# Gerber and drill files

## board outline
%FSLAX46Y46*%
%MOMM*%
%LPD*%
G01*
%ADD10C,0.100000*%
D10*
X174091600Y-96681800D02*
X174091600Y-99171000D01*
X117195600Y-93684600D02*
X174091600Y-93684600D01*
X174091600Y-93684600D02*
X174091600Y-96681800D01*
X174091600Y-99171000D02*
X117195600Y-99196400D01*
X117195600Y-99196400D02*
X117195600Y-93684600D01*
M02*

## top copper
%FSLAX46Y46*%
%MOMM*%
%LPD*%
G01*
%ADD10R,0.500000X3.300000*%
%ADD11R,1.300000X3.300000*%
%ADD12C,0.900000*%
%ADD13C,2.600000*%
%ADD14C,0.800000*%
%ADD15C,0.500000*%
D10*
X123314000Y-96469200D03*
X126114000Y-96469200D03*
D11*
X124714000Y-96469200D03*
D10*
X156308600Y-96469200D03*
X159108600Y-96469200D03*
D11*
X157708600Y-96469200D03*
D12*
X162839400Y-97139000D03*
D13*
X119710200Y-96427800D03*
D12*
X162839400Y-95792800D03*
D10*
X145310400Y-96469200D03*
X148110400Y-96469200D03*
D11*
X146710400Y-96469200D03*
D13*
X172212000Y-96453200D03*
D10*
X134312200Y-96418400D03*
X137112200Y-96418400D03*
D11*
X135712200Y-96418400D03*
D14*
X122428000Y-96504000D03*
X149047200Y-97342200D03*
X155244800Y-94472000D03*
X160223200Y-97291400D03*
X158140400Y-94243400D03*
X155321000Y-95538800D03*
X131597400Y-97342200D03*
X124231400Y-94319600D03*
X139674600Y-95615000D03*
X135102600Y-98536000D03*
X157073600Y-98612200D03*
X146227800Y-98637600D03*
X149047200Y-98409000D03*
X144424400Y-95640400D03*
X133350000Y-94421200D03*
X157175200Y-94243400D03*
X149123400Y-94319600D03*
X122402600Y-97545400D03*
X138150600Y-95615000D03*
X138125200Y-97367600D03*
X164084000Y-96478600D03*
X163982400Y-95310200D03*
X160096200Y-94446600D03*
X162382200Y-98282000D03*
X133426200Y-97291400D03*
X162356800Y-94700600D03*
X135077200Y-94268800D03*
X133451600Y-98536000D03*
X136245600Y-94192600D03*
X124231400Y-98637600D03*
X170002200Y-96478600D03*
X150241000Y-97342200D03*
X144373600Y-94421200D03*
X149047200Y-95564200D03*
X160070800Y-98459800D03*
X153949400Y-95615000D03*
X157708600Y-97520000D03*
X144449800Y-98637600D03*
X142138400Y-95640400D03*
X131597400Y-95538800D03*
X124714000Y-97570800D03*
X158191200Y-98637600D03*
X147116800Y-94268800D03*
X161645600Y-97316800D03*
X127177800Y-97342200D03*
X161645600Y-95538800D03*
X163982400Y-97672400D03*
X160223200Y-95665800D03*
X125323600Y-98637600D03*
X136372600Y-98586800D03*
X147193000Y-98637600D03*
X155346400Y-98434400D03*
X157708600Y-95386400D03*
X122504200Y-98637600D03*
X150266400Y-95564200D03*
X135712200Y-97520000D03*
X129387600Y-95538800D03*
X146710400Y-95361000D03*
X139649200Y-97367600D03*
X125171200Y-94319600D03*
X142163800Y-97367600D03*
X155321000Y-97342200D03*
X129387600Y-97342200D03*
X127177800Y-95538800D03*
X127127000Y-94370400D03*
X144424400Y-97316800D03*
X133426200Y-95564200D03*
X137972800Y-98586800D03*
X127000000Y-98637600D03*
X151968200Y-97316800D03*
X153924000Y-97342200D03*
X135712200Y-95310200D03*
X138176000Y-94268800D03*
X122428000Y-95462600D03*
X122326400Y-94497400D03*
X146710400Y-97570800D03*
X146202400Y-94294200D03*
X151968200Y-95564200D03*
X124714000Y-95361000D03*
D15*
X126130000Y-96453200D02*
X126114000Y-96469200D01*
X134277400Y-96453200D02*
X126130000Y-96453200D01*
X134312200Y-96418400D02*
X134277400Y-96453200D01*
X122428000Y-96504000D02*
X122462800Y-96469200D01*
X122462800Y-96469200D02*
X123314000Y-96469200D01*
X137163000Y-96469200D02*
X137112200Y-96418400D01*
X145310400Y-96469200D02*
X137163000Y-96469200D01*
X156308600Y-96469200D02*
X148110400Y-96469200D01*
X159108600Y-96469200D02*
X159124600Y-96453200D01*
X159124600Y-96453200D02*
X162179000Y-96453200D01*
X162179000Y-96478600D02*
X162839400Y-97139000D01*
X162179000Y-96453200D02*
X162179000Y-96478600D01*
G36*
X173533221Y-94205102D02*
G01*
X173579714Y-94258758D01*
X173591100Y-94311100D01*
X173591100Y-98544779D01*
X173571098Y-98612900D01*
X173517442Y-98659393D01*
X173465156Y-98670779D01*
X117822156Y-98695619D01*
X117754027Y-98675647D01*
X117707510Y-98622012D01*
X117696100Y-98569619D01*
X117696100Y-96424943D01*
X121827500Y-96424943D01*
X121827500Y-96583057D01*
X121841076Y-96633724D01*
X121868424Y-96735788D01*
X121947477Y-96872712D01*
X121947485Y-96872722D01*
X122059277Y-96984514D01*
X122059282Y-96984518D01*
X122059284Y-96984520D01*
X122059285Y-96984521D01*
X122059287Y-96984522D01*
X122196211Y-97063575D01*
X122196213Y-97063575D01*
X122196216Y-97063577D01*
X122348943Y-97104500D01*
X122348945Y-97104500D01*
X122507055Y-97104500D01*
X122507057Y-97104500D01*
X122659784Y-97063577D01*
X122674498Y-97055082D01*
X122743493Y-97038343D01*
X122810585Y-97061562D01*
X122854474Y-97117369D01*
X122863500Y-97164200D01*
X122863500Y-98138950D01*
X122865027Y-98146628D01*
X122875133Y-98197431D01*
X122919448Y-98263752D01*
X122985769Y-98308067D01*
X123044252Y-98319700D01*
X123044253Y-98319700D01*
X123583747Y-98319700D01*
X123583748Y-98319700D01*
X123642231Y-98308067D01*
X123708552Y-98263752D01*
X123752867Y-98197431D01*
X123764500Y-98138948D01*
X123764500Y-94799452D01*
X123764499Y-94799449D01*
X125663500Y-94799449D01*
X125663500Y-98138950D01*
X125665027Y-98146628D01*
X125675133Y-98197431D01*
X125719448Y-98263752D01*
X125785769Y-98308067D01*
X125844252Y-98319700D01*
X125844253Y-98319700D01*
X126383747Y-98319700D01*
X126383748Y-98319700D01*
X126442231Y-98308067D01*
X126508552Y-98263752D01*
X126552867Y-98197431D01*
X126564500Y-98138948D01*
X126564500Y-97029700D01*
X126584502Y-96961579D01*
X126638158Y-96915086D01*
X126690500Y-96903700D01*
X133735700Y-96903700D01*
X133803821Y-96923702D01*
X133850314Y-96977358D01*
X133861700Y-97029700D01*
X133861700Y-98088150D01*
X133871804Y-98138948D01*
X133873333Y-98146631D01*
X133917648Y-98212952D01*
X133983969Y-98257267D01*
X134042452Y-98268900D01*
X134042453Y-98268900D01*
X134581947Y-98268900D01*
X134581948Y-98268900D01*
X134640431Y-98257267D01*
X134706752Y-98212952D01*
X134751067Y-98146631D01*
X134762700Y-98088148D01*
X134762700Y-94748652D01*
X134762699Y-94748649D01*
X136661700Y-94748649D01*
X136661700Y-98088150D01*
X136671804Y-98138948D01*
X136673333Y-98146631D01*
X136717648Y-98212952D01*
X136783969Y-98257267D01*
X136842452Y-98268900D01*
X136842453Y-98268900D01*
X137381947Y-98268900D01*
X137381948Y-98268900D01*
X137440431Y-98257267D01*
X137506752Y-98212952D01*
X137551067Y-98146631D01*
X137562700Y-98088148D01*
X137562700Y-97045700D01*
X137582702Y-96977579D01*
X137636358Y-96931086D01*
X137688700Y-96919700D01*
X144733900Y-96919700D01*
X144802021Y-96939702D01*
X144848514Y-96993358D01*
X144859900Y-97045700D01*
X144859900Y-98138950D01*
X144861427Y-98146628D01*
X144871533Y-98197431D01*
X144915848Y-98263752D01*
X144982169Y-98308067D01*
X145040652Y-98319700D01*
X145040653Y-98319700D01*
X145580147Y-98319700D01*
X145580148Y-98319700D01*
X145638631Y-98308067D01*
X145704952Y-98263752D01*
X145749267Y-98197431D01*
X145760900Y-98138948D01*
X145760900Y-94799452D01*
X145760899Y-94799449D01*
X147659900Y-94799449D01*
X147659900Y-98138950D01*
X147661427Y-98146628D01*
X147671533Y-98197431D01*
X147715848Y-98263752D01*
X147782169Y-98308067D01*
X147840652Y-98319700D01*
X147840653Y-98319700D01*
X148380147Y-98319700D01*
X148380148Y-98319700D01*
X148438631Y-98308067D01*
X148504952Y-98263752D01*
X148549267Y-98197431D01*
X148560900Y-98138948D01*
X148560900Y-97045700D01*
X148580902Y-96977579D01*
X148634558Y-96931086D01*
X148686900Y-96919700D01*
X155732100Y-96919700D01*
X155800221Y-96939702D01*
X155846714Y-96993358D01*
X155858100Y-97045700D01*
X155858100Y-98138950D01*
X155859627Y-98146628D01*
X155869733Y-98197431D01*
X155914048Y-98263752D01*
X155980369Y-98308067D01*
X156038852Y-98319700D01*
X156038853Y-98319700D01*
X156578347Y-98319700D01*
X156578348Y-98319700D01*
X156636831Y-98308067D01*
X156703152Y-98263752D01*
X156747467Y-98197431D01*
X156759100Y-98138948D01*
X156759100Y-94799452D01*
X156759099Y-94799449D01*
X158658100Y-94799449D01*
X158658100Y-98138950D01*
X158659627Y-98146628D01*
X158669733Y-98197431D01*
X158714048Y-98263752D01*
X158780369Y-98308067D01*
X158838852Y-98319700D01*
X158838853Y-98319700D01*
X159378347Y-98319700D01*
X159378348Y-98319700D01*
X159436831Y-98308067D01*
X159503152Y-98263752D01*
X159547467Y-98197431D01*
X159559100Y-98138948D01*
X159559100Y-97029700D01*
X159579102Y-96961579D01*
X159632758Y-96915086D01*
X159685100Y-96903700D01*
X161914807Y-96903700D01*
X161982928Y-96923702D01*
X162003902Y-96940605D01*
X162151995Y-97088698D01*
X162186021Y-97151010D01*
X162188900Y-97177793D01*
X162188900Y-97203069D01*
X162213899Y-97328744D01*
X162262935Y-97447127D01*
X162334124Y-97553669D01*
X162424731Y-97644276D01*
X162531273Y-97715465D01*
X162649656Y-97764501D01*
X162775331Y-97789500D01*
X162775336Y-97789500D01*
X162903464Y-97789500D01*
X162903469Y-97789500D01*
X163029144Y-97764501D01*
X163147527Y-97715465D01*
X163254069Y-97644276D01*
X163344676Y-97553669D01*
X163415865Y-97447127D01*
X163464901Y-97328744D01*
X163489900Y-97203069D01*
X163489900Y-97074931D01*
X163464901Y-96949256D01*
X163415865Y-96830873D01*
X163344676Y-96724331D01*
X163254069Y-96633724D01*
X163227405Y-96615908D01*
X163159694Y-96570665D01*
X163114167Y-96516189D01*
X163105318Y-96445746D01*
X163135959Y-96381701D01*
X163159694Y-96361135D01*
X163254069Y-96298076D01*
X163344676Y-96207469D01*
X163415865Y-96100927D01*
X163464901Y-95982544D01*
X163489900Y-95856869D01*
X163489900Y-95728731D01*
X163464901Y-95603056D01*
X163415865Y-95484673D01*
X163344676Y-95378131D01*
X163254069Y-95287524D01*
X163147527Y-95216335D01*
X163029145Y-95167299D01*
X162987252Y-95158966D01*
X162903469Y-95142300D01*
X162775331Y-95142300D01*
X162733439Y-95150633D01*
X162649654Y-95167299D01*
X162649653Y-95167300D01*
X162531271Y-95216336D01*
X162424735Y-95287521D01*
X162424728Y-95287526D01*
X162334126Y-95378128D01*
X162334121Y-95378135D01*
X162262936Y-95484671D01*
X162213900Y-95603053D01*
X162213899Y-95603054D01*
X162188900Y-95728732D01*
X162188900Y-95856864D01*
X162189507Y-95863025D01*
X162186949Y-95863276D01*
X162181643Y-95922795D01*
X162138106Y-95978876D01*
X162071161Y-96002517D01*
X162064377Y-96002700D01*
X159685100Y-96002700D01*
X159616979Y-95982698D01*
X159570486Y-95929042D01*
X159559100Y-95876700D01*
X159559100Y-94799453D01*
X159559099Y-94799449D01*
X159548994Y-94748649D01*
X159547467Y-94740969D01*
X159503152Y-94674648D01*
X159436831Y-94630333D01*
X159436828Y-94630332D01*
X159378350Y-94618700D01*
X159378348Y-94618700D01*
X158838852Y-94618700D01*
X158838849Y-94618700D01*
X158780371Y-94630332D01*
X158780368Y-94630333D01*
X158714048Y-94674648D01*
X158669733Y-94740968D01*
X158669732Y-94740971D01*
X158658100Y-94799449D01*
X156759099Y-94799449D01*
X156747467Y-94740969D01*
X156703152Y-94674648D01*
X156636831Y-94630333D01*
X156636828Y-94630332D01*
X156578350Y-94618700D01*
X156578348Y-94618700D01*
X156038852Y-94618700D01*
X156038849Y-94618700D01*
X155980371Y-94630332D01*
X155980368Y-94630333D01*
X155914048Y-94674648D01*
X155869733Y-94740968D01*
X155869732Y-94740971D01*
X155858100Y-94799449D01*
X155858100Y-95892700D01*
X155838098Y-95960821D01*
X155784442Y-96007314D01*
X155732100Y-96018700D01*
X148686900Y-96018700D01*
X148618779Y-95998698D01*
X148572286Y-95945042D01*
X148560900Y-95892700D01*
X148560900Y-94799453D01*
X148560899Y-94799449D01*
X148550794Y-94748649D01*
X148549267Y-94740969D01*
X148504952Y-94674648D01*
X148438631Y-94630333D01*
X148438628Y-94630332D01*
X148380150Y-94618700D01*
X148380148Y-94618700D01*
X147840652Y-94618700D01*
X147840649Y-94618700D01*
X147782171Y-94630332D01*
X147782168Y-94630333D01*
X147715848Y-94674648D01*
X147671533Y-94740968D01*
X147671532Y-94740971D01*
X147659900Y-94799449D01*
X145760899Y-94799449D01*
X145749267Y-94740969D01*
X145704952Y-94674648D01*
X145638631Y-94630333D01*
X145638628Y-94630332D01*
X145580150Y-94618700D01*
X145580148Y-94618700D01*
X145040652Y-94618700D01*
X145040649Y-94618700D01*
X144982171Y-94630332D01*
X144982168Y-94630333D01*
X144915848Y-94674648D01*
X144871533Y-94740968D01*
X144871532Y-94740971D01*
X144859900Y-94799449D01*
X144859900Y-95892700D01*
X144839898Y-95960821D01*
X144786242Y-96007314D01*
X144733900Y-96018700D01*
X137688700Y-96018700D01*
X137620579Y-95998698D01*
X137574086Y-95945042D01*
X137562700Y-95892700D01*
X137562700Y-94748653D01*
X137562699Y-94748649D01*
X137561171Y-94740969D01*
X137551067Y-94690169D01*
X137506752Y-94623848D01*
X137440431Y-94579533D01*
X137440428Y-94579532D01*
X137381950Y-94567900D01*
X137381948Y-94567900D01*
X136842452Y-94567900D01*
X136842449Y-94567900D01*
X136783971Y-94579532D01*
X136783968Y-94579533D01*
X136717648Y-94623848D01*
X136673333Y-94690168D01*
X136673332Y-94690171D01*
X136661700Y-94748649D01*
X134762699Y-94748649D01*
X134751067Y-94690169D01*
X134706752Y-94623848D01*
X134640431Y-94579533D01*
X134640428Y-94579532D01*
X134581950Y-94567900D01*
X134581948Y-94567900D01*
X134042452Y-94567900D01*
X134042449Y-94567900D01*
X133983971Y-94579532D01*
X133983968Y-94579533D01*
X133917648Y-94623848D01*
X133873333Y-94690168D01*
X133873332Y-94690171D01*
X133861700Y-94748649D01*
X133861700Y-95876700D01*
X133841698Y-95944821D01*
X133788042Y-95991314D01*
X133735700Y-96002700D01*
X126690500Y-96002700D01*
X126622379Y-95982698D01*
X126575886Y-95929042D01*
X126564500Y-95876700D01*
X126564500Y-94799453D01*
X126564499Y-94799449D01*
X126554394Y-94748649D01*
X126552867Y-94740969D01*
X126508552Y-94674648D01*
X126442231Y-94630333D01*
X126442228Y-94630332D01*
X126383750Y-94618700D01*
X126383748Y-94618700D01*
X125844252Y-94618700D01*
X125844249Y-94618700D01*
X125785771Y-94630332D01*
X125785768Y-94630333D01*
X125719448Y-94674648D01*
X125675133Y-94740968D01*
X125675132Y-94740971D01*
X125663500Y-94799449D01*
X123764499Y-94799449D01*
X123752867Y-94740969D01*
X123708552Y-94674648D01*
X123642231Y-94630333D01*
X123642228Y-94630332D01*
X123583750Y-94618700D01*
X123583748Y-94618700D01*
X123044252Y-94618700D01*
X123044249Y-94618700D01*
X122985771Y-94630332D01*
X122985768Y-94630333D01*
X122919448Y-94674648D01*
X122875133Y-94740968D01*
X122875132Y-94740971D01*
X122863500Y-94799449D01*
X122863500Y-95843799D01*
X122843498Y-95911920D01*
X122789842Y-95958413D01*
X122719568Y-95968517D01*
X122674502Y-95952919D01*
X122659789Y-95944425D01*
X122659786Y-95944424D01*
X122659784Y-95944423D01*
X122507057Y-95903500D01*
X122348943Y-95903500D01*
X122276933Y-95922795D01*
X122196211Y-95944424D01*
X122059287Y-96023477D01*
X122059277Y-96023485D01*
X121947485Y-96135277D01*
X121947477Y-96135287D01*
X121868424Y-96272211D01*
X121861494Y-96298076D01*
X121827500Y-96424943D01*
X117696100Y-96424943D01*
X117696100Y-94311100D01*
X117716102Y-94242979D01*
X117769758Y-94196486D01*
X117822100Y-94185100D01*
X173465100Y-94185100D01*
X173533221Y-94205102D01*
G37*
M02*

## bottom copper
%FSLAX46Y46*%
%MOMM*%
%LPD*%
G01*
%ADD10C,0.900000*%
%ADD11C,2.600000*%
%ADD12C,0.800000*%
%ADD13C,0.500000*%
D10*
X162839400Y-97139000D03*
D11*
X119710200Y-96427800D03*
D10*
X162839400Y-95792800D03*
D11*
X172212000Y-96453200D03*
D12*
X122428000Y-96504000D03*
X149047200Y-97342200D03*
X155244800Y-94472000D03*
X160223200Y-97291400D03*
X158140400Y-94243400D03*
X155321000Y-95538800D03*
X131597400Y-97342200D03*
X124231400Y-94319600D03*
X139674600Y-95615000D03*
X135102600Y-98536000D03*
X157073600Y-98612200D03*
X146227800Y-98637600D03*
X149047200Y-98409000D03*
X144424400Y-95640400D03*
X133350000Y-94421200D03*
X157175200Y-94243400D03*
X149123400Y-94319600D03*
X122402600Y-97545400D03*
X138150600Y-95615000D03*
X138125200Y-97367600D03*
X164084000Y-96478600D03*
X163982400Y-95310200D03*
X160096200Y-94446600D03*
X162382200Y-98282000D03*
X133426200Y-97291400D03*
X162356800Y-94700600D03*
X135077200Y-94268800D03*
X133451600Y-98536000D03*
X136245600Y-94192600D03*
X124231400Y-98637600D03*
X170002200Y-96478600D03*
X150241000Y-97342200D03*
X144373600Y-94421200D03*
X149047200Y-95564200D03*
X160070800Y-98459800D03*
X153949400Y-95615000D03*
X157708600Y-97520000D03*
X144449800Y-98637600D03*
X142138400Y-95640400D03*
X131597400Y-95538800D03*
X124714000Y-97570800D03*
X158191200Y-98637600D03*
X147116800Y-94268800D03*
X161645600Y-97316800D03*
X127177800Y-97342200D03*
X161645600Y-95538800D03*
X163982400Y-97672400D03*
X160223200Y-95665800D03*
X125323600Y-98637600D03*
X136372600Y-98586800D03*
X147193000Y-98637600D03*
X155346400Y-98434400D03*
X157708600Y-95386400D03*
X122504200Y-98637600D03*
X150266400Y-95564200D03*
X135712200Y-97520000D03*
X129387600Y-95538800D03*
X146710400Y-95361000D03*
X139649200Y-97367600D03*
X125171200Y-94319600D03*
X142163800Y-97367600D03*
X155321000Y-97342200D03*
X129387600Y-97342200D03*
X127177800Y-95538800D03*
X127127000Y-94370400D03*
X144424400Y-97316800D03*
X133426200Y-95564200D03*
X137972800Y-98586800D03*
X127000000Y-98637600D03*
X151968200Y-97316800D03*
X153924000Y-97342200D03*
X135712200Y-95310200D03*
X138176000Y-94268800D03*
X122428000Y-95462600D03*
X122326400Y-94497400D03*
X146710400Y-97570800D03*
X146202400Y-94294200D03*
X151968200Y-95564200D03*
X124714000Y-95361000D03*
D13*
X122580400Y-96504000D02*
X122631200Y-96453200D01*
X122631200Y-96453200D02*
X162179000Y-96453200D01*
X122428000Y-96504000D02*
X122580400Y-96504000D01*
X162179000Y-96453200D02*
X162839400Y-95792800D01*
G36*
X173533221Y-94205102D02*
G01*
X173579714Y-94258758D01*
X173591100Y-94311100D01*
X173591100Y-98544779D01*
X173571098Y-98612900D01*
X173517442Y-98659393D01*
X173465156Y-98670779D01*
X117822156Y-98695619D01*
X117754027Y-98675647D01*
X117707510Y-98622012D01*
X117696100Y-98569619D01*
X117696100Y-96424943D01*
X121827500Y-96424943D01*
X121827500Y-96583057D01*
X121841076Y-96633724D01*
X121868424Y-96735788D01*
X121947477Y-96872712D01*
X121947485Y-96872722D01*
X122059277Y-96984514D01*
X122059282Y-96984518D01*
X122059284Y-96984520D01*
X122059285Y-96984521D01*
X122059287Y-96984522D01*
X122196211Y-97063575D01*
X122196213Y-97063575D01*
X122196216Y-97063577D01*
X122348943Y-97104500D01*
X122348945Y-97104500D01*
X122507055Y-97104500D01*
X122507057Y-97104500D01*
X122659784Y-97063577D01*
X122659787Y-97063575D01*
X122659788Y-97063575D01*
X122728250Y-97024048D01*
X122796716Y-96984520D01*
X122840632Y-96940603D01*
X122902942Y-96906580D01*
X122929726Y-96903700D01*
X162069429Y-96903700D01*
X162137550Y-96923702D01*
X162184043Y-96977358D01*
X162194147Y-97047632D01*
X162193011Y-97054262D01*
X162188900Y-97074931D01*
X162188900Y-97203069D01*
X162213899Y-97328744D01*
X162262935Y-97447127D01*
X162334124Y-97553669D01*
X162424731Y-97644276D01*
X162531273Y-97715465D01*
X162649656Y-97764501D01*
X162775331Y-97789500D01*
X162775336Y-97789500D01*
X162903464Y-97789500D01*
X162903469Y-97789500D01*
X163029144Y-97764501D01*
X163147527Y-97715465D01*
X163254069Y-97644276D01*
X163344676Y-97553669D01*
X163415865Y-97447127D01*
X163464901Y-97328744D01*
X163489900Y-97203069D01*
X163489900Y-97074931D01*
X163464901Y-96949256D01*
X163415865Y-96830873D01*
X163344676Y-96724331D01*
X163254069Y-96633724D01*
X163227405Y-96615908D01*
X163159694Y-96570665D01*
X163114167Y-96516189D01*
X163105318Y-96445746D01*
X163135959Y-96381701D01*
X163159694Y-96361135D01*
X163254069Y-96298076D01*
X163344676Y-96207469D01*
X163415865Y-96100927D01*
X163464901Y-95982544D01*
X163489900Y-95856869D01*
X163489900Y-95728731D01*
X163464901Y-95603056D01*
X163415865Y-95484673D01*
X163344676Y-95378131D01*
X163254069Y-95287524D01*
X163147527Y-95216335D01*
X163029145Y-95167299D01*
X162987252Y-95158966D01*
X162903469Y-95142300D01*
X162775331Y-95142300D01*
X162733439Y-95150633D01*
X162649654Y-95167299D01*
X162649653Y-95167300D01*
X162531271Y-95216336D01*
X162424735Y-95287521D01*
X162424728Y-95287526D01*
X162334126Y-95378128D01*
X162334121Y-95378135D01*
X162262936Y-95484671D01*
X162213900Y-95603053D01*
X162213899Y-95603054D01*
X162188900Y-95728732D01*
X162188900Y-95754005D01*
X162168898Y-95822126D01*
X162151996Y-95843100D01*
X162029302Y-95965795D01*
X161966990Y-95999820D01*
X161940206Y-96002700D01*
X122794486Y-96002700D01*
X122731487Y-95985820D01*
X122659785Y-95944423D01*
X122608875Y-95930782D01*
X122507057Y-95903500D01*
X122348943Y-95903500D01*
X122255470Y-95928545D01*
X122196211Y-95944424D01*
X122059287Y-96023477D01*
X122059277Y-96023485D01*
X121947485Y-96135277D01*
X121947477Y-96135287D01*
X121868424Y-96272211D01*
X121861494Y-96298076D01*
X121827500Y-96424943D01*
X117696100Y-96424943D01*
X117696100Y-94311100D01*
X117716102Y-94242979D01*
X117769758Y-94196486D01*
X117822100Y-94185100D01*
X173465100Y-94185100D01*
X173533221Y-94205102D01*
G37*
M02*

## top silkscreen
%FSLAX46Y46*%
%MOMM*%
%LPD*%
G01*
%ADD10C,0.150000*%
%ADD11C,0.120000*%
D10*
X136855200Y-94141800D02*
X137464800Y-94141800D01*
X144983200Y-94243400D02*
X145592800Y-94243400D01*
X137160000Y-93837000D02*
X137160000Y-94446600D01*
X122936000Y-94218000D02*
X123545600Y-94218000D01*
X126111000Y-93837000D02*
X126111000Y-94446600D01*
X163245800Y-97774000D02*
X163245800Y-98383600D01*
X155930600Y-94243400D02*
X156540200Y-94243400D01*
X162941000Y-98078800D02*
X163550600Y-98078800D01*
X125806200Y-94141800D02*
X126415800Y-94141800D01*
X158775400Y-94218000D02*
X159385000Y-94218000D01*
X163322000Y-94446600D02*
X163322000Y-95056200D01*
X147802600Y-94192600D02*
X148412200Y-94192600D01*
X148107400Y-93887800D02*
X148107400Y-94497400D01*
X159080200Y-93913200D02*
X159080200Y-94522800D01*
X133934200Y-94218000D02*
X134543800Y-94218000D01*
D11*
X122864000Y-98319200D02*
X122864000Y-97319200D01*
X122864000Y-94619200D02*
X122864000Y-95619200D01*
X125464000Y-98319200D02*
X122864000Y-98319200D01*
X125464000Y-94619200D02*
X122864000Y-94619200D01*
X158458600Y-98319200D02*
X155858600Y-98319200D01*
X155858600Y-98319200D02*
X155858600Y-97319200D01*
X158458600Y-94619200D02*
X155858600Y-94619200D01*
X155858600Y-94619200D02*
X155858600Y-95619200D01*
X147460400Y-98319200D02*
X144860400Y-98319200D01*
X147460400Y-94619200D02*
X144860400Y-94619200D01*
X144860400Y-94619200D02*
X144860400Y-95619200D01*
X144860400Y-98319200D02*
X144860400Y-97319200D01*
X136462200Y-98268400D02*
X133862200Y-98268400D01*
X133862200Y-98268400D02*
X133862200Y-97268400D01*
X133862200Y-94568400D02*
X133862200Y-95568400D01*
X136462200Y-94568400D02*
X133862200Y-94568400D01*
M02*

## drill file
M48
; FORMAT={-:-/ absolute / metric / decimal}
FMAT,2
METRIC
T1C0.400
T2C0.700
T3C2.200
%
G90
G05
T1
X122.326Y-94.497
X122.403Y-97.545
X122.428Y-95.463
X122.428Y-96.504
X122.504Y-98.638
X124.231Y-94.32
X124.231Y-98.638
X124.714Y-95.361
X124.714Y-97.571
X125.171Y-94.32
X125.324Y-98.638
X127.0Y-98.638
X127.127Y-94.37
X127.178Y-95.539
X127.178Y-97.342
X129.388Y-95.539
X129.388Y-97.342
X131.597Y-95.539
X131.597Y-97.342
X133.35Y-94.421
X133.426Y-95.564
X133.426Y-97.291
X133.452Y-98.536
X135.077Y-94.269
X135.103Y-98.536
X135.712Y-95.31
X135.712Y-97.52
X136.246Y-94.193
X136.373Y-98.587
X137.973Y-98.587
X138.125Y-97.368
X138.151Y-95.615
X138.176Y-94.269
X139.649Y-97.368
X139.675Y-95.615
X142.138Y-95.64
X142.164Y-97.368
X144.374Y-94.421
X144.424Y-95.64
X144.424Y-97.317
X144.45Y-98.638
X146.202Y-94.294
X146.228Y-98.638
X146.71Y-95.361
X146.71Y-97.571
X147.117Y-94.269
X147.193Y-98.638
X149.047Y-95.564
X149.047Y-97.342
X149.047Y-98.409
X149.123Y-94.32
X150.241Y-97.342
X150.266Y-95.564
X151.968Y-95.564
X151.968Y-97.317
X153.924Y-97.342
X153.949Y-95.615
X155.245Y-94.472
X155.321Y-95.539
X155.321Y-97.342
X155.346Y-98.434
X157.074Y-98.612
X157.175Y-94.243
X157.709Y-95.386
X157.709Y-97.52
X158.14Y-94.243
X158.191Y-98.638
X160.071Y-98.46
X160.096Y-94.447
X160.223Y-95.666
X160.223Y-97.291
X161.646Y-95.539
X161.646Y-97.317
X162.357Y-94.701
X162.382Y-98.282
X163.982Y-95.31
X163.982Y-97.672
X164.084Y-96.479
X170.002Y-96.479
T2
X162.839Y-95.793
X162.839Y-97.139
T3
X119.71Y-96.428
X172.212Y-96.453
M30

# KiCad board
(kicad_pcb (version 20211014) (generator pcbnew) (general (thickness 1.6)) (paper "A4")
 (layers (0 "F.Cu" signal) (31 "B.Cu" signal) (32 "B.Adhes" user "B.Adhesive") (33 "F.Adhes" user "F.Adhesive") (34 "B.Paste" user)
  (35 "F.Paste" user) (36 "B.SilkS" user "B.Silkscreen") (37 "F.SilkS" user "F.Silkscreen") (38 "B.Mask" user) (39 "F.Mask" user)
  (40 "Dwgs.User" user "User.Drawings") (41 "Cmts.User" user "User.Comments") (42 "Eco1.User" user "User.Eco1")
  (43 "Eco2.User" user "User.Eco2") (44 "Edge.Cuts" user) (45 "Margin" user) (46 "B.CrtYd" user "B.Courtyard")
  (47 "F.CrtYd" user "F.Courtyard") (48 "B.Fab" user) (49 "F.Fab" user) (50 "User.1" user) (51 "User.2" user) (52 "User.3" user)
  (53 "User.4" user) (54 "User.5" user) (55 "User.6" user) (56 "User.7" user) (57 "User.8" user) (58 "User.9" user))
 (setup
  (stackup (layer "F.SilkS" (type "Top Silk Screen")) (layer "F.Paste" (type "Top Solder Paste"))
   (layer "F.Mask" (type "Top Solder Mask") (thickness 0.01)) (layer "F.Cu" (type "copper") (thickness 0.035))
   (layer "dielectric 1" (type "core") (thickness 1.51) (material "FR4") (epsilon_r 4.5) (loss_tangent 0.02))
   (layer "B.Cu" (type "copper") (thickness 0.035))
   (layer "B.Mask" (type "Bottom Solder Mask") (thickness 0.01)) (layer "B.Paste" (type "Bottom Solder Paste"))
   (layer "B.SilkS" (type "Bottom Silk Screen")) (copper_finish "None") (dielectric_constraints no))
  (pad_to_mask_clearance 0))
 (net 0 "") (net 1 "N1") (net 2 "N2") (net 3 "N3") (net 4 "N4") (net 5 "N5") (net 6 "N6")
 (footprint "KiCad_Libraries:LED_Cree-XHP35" (layer "F.Cu") (at 124.714 96.4692)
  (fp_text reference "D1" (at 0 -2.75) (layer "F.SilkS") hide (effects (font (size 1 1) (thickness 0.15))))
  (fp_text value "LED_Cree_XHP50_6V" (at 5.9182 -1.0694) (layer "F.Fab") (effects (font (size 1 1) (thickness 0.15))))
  (fp_line (start -1.85 1.85) (end -1.85 0.85) (layer "F.SilkS") (width 0.12))
  (fp_line (start -1.85 -1.85) (end -1.85 -0.85) (layer "F.SilkS") (width 0.12))
  (fp_line (start 0.75 1.85) (end -1.85 1.85) (layer "F.SilkS") (width 0.12))
  (fp_line (start 0.75 -1.85) (end -1.85 -1.85) (layer "F.SilkS") (width 0.12))
  (pad "" smd rect locked (at 0 -1) (size 1.01 0.75) (layers "F.Paste"))
  (pad "" smd rect locked (at 0 1) (size 1.01 0.75) (layers "F.Paste"))
  (pad "" smd rect locked (at 0 0) (size 1.01 0.75) (layers "F.Paste"))
  (pad "1" smd rect locked (at -1.4 0) (size 0.5 3.3) (layers "F.Cu" "F.Paste" "F.Mask") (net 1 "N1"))
  (pad "2" smd rect locked (at 1.4 0) (size 0.5 3.3) (layers "F.Cu" "F.Paste" "F.Mask") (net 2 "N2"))
  (pad "3" smd rect locked (at 0 0) (size 1.3 3.3) (layers "F.Cu" "F.Mask") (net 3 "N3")))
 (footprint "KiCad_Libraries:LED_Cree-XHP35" (layer "F.Cu") (at 157.7086 96.4692)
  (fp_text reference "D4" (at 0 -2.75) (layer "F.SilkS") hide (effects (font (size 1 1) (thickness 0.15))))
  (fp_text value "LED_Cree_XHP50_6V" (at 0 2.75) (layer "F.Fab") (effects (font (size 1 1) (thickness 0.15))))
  (fp_line (start 0.75 1.85) (end -1.85 1.85) (layer "F.SilkS") (width 0.12))
  (fp_line (start -1.85 1.85) (end -1.85 0.85) (layer "F.SilkS") (width 0.12))
  (fp_line (start 0.75 -1.85) (end -1.85 -1.85) (layer "F.SilkS") (width 0.12))
  (fp_line (start -1.85 -1.85) (end -1.85 -0.85) (layer "F.SilkS") (width 0.12))
  (pad "" smd rect locked (at 0 -1) (size 1.01 0.75) (layers "F.Paste"))
  (pad "" smd rect locked (at 0 0) (size 1.01 0.75) (layers "F.Paste"))
  (pad "" smd rect locked (at 0 1) (size 1.01 0.75) (layers "F.Paste"))
  (pad "1" smd rect locked (at -1.4 0) (size 0.5 3.3) (layers "F.Cu" "F.Paste" "F.Mask") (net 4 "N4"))
  (pad "2" smd rect locked (at 1.4 0) (size 0.5 3.3) (layers "F.Cu" "F.Paste" "F.Mask") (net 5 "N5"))
  (pad "3" smd rect locked (at 0 0) (size 1.3 3.3) (layers "F.Cu" "F.Mask") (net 3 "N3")))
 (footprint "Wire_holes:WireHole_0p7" (layer "F.Cu") (at 162.8394 97.139)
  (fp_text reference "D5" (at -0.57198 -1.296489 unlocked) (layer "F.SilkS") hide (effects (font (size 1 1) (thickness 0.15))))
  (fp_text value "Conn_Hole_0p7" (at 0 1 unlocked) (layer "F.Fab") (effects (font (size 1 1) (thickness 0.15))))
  (pad "1" thru_hole circle (at 0 0) (size 0.9 0.9) (drill 0.7) (layers *.Cu *.Mask) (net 5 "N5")))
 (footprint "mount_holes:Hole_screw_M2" (layer "F.Cu") (at 119.7102 96.4278)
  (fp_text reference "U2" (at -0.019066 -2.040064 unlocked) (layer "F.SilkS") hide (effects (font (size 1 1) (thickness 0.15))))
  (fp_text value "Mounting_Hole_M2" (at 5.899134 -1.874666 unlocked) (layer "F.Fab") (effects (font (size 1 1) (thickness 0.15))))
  (pad "1" thru_hole circle (at 0 0) (size 2.6 2.6) (drill 2.2) (layers *.Cu *.Mask) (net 3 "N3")))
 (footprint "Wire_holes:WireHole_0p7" (layer "F.Cu") (at 162.8394 95.7928)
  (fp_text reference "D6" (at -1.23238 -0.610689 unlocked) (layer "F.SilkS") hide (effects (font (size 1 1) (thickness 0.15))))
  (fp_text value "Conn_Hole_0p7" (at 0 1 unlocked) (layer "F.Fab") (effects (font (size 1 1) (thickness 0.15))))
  (pad "1" thru_hole circle (at 0 0) (size 0.9 0.9) (drill 0.7) (layers *.Cu *.Mask) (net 1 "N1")))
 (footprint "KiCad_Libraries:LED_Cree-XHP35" (layer "F.Cu") (at 146.7104 96.4692)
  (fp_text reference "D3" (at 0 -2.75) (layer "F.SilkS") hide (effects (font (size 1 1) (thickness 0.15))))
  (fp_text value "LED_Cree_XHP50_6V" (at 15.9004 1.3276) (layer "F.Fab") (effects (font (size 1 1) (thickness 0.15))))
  (fp_line (start 0.75 1.85) (end -1.85 1.85) (layer "F.SilkS") (width 0.12))
  (fp_line (start 0.75 -1.85) (end -1.85 -1.85) (layer "F.SilkS") (width 0.12))
  (fp_line (start -1.85 -1.85) (end -1.85 -0.85) (layer "F.SilkS") (width 0.12))
  (fp_line (start -1.85 1.85) (end -1.85 0.85) (layer "F.SilkS") (width 0.12))
  (pad "" smd rect locked (at 0 1) (size 1.01 0.75) (layers "F.Paste"))
  (pad "" smd rect locked (at 0 -1) (size 1.01 0.75) (layers "F.Paste"))
  (pad "" smd rect locked (at 0 0) (size 1.01 0.75) (layers "F.Paste"))
  (pad "1" smd rect locked (at -1.4 0) (size 0.5 3.3) (layers "F.Cu" "F.Paste" "F.Mask") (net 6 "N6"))
  (pad "2" smd rect locked (at 1.4 0) (size 0.5 3.3) (layers "F.Cu" "F.Paste" "F.Mask") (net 4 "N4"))
  (pad "3" smd rect locked (at 0 0) (size 1.3 3.3) (layers "F.Cu" "F.Mask") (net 3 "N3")))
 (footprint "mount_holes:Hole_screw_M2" (layer "F.Cu") (at 172.212 96.4532)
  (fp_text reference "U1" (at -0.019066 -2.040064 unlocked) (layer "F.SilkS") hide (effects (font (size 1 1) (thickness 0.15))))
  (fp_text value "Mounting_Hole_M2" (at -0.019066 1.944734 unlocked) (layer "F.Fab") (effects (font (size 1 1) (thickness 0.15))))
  (pad "1" thru_hole circle (at 0 0) (size 2.6 2.6) (drill 2.2) (layers *.Cu *.Mask) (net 3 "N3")))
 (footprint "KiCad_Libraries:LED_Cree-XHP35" (layer "F.Cu") (at 135.7122 96.4184)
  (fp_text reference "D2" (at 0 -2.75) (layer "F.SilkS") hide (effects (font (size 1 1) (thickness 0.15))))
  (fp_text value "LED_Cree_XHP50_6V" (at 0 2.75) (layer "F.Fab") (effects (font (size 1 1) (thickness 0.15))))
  (fp_line (start 0.75 1.85) (end -1.85 1.85) (layer "F.SilkS") (width 0.12))
  (fp_line (start -1.85 1.85) (end -1.85 0.85) (layer "F.SilkS") (width 0.12))
  (fp_line (start -1.85 -1.85) (end -1.85 -0.85) (layer "F.SilkS") (width 0.12))
  (fp_line (start 0.75 -1.85) (end -1.85 -1.85) (layer "F.SilkS") (width 0.12))
  (pad "" smd rect locked (at 0 -1) (size 1.01 0.75) (layers "F.Paste"))
  (pad "" smd rect locked (at 0 1) (size 1.01 0.75) (layers "F.Paste"))
  (pad "" smd rect locked (at 0 0) (size 1.01 0.75) (layers "F.Paste"))
  (pad "1" smd rect locked (at -1.4 0) (size 0.5 3.3) (layers "F.Cu" "F.Paste" "F.Mask") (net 2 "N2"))
  (pad "2" smd rect locked (at 1.4 0) (size 0.5 3.3) (layers "F.Cu" "F.Paste" "F.Mask") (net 6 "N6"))
  (pad "3" smd rect locked (at 0 0) (size 1.3 3.3) (layers "F.Cu" "F.Mask") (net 3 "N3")))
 (gr_line (start 136.8552 94.1418) (end 137.4648 94.1418) (layer "F.SilkS") (width 0.15))
 (gr_line (start 144.9832 94.2434) (end 145.5928 94.2434) (layer "F.SilkS") (width 0.15))
 (gr_line (start 137.16 93.837) (end 137.16 94.4466) (layer "F.SilkS") (width 0.15))
 (gr_line (start 122.936 94.218) (end 123.5456 94.218) (layer "F.SilkS") (width 0.15))
 (gr_line (start 126.111 93.837) (end 126.111 94.4466) (layer "F.SilkS") (width 0.15))
 (gr_line (start 163.2458 97.774) (end 163.2458 98.3836) (layer "F.SilkS") (width 0.15))
 (gr_line (start 155.9306 94.2434) (end 156.5402 94.2434) (layer "F.SilkS") (width 0.15))
 (gr_line (start 162.941 98.0788) (end 163.5506 98.0788) (layer "F.SilkS") (width 0.15))
 (gr_line (start 125.8062 94.1418) (end 126.4158 94.1418) (layer "F.SilkS") (width 0.15))
 (gr_line (start 158.7754 94.218) (end 159.385 94.218) (layer "F.SilkS") (width 0.15))
 (gr_line (start 163.322 94.4466) (end 163.322 95.0562) (layer "F.SilkS") (width 0.15))
 (gr_line (start 147.8026 94.1926) (end 148.4122 94.1926) (layer "F.SilkS") (width 0.15))
 (gr_line (start 148.1074 93.8878) (end 148.1074 94.4974) (layer "F.SilkS") (width 0.15))
 (gr_line (start 159.0802 93.9132) (end 159.0802 94.5228) (layer "F.SilkS") (width 0.15))
 (gr_line (start 133.9342 94.218) (end 134.5438 94.218) (layer "F.SilkS") (width 0.15))
 (gr_line (start 174.0916 96.6818) (end 174.0916 99.171) (layer "Edge.Cuts") (width 0.1))
 (gr_line (start 117.1956 93.6846) (end 174.0916 93.6846) (layer "Edge.Cuts") (width 0.1))
 (gr_line (start 174.0916 93.6846) (end 174.0916 96.6818) (layer "Edge.Cuts") (width 0.1))
 (gr_line (start 174.0916 99.171) (end 117.1956 99.1964) (layer "Edge.Cuts") (width 0.1))
 (gr_line (start 117.1956 99.1964) (end 117.1956 93.6846) (layer "Edge.Cuts") (width 0.1))
 (segment (start 126.13 96.4532) (end 126.114 96.4692) (width 0.5) (layer "F.Cu") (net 2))
 (segment (start 134.2774 96.4532) (end 126.13 96.4532) (width 0.5) (layer "F.Cu") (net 2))
 (segment (start 134.3122 96.4184) (end 134.2774 96.4532) (width 0.5) (layer "F.Cu") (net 2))
 (segment (start 122.428 96.504) (end 122.4628 96.4692) (width 0.5) (layer "F.Cu") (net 1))
 (segment (start 122.4628 96.4692) (end 123.314 96.4692) (width 0.5) (layer "F.Cu") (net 1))
 (via (at 122.428 96.504) (size 0.8) (drill 0.4) (layers "F.Cu" "B.Cu") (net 1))
 (segment (start 122.5804 96.504) (end 122.6312 96.4532) (width 0.5) (layer "B.Cu") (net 1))
 (segment (start 122.6312 96.4532) (end 162.179 96.4532) (width 0.5) (layer "B.Cu") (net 1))
 (segment (start 122.428 96.504) (end 122.5804 96.504) (width 0.5) (layer "B.Cu") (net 1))
 (segment (start 162.179 96.4532) (end 162.8394 95.7928) (width 0.5) (layer "B.Cu") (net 1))
 (via (at 149.0472 97.3422) (size 0.8) (drill 0.4) (layers "F.Cu" "B.Cu") (free) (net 3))
 (via (at 155.2448 94.472) (size 0.8) (drill 0.4) (layers "F.Cu" "B.Cu") (free) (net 3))
 (via (at 160.2232 97.2914) (size 0.8) (drill 0.4) (layers "F.Cu" "B.Cu") (free) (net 3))
 (via (at 158.1404 94.2434) (size 0.8) (drill 0.4) (layers "F.Cu" "B.Cu") (free) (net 3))
 (via (at 155.321 95.5388) (size 0.8) (drill 0.4) (layers "F.Cu" "B.Cu") (free) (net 3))
 (via (at 131.5974 97.3422) (size 0.8) (drill 0.4) (layers "F.Cu" "B.Cu") (free) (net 3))
 (via (at 124.2314 94.3196) (size 0.8) (drill 0.4) (layers "F.Cu" "B.Cu") (free) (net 3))
 (via (at 139.6746 95.615) (size 0.8) (drill 0.4) (layers "F.Cu" "B.Cu") (free) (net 3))
 (via (at 135.1026 98.536) (size 0.8) (drill 0.4) (layers "F.Cu" "B.Cu") (free) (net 3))
 (via (at 157.0736 98.6122) (size 0.8) (drill 0.4) (layers "F.Cu" "B.Cu") (free) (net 3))
 (via (at 146.2278 98.6376) (size 0.8) (drill 0.4) (layers "F.Cu" "B.Cu") (free) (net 3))
 (via (at 149.0472 98.409) (size 0.8) (drill 0.4) (layers "F.Cu" "B.Cu") (free) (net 3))
 (via (at 144.4244 95.6404) (size 0.8) (drill 0.4) (layers "F.Cu" "B.Cu") (free) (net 3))
 (via (at 133.35 94.4212) (size 0.8) (drill 0.4) (layers "F.Cu" "B.Cu") (free) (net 3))
 (via (at 157.1752 94.2434) (size 0.8) (drill 0.4) (layers "F.Cu" "B.Cu") (free) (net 3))
 (via (at 149.1234 94.3196) (size 0.8) (drill 0.4) (layers "F.Cu" "B.Cu") (free) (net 3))
 (via (at 122.4026 97.5454) (size 0.8) (drill 0.4) (layers "F.Cu" "B.Cu") (free) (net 3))
 (via (at 138.1506 95.615) (size 0.8) (drill 0.4) (layers "F.Cu" "B.Cu") (free) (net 3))
 (via (at 138.1252 97.3676) (size 0.8) (drill 0.4) (layers "F.Cu" "B.Cu") (free) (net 3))
 (via (at 164.084 96.4786) (size 0.8) (drill 0.4) (layers "F.Cu" "B.Cu") (free) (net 3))
 (via (at 163.9824 95.3102) (size 0.8) (drill 0.4) (layers "F.Cu" "B.Cu") (free) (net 3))
 (via (at 160.0962 94.4466) (size 0.8) (drill 0.4) (layers "F.Cu" "B.Cu") (free) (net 3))
 (via (at 162.3822 98.282) (size 0.8) (drill 0.4) (layers "F.Cu" "B.Cu") (free) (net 3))
 (via (at 133.4262 97.2914) (size 0.8) (drill 0.4) (layers "F.Cu" "B.Cu") (free) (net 3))
 (via (at 162.3568 94.7006) (size 0.8) (drill 0.4) (layers "F.Cu" "B.Cu") (free) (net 3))
 (via (at 135.0772 94.2688) (size 0.8) (drill 0.4) (layers "F.Cu" "B.Cu") (free) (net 3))
 (via (at 133.4516 98.536) (size 0.8) (drill 0.4) (layers "F.Cu" "B.Cu") (free) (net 3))
 (via (at 136.2456 94.1926) (size 0.8) (drill 0.4) (layers "F.Cu" "B.Cu") (free) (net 3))
 (via (at 124.2314 98.6376) (size 0.8) (drill 0.4) (layers "F.Cu" "B.Cu") (free) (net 3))
 (via (at 170.0022 96.4786) (size 0.8) (drill 0.4) (layers "F.Cu" "B.Cu") (free) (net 3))
 (via (at 150.241 97.3422) (size 0.8) (drill 0.4) (layers "F.Cu" "B.Cu") (free) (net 3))
 (via (at 144.3736 94.4212) (size 0.8) (drill 0.4) (layers "F.Cu" "B.Cu") (free) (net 3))
 (via (at 149.0472 95.5642) (size 0.8) (drill 0.4) (layers "F.Cu" "B.Cu") (free) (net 3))
 (via (at 160.0708 98.4598) (size 0.8) (drill 0.4) (layers "F.Cu" "B.Cu") (free) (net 3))
 (via (at 153.9494 95.615) (size 0.8) (drill 0.4) (layers "F.Cu" "B.Cu") (free) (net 3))
 (via (at 157.7086 97.52) (size 0.8) (drill 0.4) (layers "F.Cu" "B.Cu") (free) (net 3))
 (via (at 144.4498 98.6376) (size 0.8) (drill 0.4) (layers "F.Cu" "B.Cu") (free) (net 3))
 (via (at 142.1384 95.6404) (size 0.8) (drill 0.4) (layers "F.Cu" "B.Cu") (free) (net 3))
 (via (at 131.5974 95.5388) (size 0.8) (drill 0.4) (layers "F.Cu" "B.Cu") (free) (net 3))
 (via (at 124.714 97.5708) (size 0.8) (drill 0.4) (layers "F.Cu" "B.Cu") (free) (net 3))
 (via (at 158.1912 98.6376) (size 0.8) (drill 0.4) (layers "F.Cu" "B.Cu") (free) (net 3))
 (via (at 147.1168 94.2688) (size 0.8) (drill 0.4) (layers "F.Cu" "B.Cu") (free) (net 3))
 (via (at 161.6456 97.3168) (size 0.8) (drill 0.4) (layers "F.Cu" "B.Cu") (free) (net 3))
 (via (at 127.1778 97.3422) (size 0.8) (drill 0.4) (layers "F.Cu" "B.Cu") (free) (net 3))
 (via (at 161.6456 95.5388) (size 0.8) (drill 0.4) (layers "F.Cu" "B.Cu") (free) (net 3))
 (via (at 163.9824 97.6724) (size 0.8) (drill 0.4) (layers "F.Cu" "B.Cu") (free) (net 3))
 (via (at 160.2232 95.6658) (size 0.8) (drill 0.4) (layers "F.Cu" "B.Cu") (free) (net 3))
 (via (at 125.3236 98.6376) (size 0.8) (drill 0.4) (layers "F.Cu" "B.Cu") (free) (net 3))
 (via (at 136.3726 98.5868) (size 0.8) (drill 0.4) (layers "F.Cu" "B.Cu") (free) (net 3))
 (via (at 147.193 98.6376) (size 0.8) (drill 0.4) (layers "F.Cu" "B.Cu") (free) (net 3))
 (via (at 155.3464 98.4344) (size 0.8) (drill 0.4) (layers "F.Cu" "B.Cu") (free) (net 3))
 (via (at 157.7086 95.3864) (size 0.8) (drill 0.4) (layers "F.Cu" "B.Cu") (free) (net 3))
 (via (at 122.5042 98.6376) (size 0.8) (drill 0.4) (layers "F.Cu" "B.Cu") (free) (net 3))
 (via (at 150.2664 95.5642) (size 0.8) (drill 0.4) (layers "F.Cu" "B.Cu") (free) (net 3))
 (via (at 135.7122 97.52) (size 0.8) (drill 0.4) (layers "F.Cu" "B.Cu") (free) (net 3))
 (via (at 129.3876 95.5388) (size 0.8) (drill 0.4) (layers "F.Cu" "B.Cu") (free) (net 3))
 (via (at 146.7104 95.361) (size 0.8) (drill 0.4) (layers "F.Cu" "B.Cu") (free) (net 3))
 (via (at 139.6492 97.3676) (size 0.8) (drill 0.4) (layers "F.Cu" "B.Cu") (free) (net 3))
 (via (at 125.1712 94.3196) (size 0.8) (drill 0.4) (layers "F.Cu" "B.Cu") (free) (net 3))
 (via (at 142.1638 97.3676) (size 0.8) (drill 0.4) (layers "F.Cu" "B.Cu") (free) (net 3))
 (via (at 155.321 97.3422) (size 0.8) (drill 0.4) (layers "F.Cu" "B.Cu") (free) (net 3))
 (via (at 129.3876 97.3422) (size 0.8) (drill 0.4) (layers "F.Cu" "B.Cu") (free) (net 3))
 (via (at 127.1778 95.5388) (size 0.8) (drill 0.4) (layers "F.Cu" "B.Cu") (free) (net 3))
 (via (at 127.127 94.3704) (size 0.8) (drill 0.4) (layers "F.Cu" "B.Cu") (free) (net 3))
 (via (at 144.4244 97.3168) (size 0.8) (drill 0.4) (layers "F.Cu" "B.Cu") (free) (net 3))
 (via (at 133.4262 95.5642) (size 0.8) (drill 0.4) (layers "F.Cu" "B.Cu") (free) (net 3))
 (via (at 137.9728 98.5868) (size 0.8) (drill 0.4) (layers "F.Cu" "B.Cu") (free) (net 3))
 (via (at 127 98.6376) (size 0.8) (drill 0.4) (layers "F.Cu" "B.Cu") (free) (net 3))
 (via (at 151.9682 97.3168) (size 0.8) (drill 0.4) (layers "F.Cu" "B.Cu") (free) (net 3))
 (via (at 153.924 97.3422) (size 0.8) (drill 0.4) (layers "F.Cu" "B.Cu") (free) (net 3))
 (via (at 135.7122 95.3102) (size 0.8) (drill 0.4) (layers "F.Cu" "B.Cu") (free) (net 3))
 (via (at 138.176 94.2688) (size 0.8) (drill 0.4) (layers "F.Cu" "B.Cu") (free) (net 3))
 (via (at 122.428 95.4626) (size 0.8) (drill 0.4) (layers "F.Cu" "B.Cu") (free) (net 3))
 (via (at 122.3264 94.4974) (size 0.8) (drill 0.4) (layers "F.Cu" "B.Cu") (free) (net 3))
 (via (at 146.7104 97.5708) (size 0.8) (drill 0.4) (layers "F.Cu" "B.Cu") (free) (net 3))
 (via (at 146.2024 94.2942) (size 0.8) (drill 0.4) (layers "F.Cu" "B.Cu") (free) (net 3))
 (via (at 151.9682 95.5642) (size 0.8) (drill 0.4) (layers "F.Cu" "B.Cu") (free) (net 3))
 (via (at 124.714 95.361) (size 0.8) (drill 0.4) (layers "F.Cu" "B.Cu") (free) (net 3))
 (segment (start 137.163 96.4692) (end 137.1122 96.4184) (width 0.5) (layer "F.Cu") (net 6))
 (segment (start 145.3104 96.4692) (end 137.163 96.4692) (width 0.5) (layer "F.Cu") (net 6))
 (segment (start 156.3086 96.4692) (end 148.1104 96.4692) (width 0.5) (layer "F.Cu") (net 4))
 (segment (start 159.1086 96.4692) (end 159.1246 96.4532) (width 0.5) (layer "F.Cu") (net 5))
 (segment (start 159.1246 96.4532) (end 162.179 96.4532) (width 0.5) (layer "F.Cu") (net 5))
 (segment (start 162.179 96.4786) (end 162.8394 97.139) (width 0.5) (layer "F.Cu") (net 5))
 (segment (start 162.179 96.4532) (end 162.179 96.4786) (width 0.5) (layer "F.Cu") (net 5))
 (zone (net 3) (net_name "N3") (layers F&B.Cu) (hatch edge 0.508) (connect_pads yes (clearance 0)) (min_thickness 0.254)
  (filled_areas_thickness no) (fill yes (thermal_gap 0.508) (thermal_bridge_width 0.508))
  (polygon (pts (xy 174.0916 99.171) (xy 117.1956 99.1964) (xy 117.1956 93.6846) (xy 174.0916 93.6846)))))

